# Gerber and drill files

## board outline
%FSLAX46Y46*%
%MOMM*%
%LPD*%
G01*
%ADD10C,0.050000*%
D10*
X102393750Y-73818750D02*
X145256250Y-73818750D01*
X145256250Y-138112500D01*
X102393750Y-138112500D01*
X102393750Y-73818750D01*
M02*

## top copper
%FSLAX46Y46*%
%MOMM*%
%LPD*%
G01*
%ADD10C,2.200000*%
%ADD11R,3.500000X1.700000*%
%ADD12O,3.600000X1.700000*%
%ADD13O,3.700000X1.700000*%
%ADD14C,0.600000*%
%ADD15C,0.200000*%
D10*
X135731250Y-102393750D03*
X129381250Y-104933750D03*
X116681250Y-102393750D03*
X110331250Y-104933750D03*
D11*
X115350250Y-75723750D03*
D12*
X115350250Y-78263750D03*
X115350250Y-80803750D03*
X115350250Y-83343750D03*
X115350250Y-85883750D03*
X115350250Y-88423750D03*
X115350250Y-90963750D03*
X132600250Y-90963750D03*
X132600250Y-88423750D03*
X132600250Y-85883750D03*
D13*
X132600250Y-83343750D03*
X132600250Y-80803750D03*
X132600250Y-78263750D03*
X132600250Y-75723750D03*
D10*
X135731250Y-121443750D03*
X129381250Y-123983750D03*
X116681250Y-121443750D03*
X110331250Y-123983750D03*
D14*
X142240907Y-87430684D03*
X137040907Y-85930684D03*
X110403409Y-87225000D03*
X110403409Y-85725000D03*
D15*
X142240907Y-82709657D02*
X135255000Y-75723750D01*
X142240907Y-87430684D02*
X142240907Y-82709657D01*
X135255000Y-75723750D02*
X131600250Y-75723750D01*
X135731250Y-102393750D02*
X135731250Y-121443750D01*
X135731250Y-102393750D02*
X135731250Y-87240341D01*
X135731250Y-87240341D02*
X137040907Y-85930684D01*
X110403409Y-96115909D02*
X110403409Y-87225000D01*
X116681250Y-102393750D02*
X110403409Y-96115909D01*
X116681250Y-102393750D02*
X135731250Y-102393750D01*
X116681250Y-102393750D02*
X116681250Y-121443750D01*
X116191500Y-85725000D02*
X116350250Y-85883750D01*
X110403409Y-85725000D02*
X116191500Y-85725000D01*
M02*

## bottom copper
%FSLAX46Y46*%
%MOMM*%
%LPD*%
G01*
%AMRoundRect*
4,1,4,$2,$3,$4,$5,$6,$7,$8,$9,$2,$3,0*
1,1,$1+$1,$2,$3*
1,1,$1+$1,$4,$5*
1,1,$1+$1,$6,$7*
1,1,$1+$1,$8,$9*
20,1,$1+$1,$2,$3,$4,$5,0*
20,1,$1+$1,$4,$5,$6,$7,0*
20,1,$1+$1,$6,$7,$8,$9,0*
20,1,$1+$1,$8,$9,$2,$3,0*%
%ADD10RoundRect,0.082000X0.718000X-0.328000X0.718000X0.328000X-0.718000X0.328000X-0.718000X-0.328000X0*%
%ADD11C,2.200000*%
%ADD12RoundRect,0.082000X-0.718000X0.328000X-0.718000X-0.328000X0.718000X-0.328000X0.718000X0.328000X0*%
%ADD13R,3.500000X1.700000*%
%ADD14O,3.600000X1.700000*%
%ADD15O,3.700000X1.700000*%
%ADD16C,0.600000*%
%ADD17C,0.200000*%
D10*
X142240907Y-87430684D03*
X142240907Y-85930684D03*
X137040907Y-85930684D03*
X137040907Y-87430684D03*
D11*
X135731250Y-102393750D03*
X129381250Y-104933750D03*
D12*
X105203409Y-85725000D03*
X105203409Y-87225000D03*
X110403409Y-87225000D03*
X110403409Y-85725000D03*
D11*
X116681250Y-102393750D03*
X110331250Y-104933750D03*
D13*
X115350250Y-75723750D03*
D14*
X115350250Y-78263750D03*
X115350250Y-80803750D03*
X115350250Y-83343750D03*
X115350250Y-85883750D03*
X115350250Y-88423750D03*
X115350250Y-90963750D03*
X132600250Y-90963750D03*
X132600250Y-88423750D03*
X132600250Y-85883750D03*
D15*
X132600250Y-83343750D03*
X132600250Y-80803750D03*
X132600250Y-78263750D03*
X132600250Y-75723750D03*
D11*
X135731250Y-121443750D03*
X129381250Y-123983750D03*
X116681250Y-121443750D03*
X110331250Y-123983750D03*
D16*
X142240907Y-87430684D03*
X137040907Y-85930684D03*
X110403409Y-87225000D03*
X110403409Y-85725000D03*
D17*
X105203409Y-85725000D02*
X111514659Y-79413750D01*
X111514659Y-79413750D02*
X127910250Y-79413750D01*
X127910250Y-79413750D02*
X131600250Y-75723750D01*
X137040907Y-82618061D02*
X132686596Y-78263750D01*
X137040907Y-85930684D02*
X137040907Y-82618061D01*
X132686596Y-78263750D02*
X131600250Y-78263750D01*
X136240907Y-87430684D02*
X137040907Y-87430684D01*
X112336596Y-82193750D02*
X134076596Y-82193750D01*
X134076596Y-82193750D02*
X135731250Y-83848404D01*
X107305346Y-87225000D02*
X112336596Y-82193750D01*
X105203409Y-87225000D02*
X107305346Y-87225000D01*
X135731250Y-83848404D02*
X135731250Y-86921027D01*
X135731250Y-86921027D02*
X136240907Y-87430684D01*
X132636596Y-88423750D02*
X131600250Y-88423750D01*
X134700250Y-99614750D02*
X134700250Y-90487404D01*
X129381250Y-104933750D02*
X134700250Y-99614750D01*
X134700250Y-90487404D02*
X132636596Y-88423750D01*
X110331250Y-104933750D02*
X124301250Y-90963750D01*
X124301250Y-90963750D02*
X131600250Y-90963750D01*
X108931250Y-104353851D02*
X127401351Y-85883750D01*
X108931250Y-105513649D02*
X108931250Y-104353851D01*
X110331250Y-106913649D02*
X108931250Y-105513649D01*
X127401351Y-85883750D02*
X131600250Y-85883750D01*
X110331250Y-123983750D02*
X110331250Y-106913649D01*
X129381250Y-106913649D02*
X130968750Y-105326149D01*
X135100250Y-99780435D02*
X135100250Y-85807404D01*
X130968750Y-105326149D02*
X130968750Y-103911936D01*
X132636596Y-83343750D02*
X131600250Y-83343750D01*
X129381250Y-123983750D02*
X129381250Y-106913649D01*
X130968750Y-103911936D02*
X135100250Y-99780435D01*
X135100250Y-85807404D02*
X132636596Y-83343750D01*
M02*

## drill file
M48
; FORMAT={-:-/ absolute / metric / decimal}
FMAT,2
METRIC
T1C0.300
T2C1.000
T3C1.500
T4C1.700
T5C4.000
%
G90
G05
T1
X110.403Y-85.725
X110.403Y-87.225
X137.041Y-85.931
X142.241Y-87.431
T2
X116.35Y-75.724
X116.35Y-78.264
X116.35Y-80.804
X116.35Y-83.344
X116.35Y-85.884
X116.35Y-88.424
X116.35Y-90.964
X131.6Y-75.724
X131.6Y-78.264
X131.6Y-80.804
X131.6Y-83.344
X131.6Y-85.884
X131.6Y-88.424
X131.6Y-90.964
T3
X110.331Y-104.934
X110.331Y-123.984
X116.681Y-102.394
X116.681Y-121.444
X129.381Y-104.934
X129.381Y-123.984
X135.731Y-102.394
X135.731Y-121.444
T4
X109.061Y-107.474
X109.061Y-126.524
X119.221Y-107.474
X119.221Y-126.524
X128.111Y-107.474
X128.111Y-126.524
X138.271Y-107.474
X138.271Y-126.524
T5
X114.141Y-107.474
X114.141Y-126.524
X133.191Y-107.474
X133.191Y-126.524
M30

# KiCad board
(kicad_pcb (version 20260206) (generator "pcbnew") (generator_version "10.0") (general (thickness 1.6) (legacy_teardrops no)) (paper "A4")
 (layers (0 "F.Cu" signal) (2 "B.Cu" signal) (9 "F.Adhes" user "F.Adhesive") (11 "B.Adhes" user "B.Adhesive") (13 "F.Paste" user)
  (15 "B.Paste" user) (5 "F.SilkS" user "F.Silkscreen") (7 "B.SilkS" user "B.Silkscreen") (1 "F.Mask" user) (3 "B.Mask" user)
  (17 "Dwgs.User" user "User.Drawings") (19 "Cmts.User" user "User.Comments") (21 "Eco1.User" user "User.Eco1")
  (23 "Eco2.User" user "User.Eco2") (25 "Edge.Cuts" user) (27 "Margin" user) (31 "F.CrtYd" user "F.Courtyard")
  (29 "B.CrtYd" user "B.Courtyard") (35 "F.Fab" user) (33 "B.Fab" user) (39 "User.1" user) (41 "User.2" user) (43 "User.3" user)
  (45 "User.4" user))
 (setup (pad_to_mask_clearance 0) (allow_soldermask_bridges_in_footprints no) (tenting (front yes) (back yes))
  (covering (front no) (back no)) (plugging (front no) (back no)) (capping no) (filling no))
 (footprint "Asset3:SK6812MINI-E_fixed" (layer "F.Cu") (at 139.640908 86.577842 180)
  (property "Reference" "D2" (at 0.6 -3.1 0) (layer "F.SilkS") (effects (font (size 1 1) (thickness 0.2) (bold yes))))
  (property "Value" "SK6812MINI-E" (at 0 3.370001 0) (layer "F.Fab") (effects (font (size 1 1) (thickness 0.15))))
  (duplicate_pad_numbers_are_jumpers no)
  (pad "1" smd roundrect (at -2.599999 -0.852842 90) (size 0.82 1.6) (layers "B.Cu" "B.Mask" "B.Paste") (roundrect_rratio 0.1) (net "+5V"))
  (pad "2" smd roundrect (at -2.599999 0.647158 90) (size 0.82 1.6) (layers "B.Cu" "B.Mask" "B.Paste") (roundrect_rratio 0.1)
   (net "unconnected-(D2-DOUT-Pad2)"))
  (pad "3" smd roundrect (at 2.600001 0.647158 90) (size 0.82 1.6) (layers "B.Cu" "B.Mask" "B.Paste") (roundrect_rratio 0.1) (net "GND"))
  (pad "4" smd roundrect (at 2.600001 -0.852842 90) (size 0.82 1.6) (layers "B.Cu" "B.Mask" "B.Paste") (roundrect_rratio 0.1)
   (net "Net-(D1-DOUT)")))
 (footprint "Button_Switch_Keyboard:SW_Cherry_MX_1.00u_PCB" (layer "F.Cu") (at 135.73125 102.39375)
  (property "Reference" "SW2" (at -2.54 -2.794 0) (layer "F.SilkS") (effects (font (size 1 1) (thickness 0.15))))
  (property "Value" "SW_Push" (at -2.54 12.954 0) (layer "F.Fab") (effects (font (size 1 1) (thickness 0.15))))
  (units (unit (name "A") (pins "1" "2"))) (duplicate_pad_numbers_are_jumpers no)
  (pad "" np_thru_hole circle (at -7.62 5.08) (size 1.7 1.7) (drill 1.7) (layers "*.Cu" "*.Mask"))
  (pad "" np_thru_hole circle (at -2.54 5.08) (size 4 4) (drill 4) (layers "*.Cu" "*.Mask"))
  (pad "" np_thru_hole circle (at 2.54 5.08) (size 1.7 1.7) (drill 1.7) (layers "*.Cu" "*.Mask"))
  (pad "1" thru_hole circle (at 0 0) (size 2.2 2.2) (drill 1.5) (layers "*.Cu" "*.Mask") (remove_unused_layers no) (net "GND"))
  (pad "2" thru_hole circle (at -6.35 2.54) (size 2.2 2.2) (drill 1.5) (layers "*.Cu" "*.Mask") (remove_unused_layers no)
   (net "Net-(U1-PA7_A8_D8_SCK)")))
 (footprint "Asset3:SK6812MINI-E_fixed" (layer "F.Cu") (at 107.803408 86.577842)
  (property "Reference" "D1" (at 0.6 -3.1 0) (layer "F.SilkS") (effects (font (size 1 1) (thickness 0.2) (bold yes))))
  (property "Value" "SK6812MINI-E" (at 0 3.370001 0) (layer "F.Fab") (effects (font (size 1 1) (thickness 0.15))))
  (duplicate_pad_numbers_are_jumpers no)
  (pad "1" smd roundrect (at -2.599999 -0.852842 270) (size 0.82 1.6) (layers "B.Cu" "B.Mask" "B.Paste") (roundrect_rratio 0.1) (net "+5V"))
  (pad "2" smd roundrect (at -2.599999 0.647158 270) (size 0.82 1.6) (layers "B.Cu" "B.Mask" "B.Paste") (roundrect_rratio 0.1)
   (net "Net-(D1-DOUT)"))
  (pad "3" smd roundrect (at 2.600001 0.647158 270) (size 0.82 1.6) (layers "B.Cu" "B.Mask" "B.Paste") (roundrect_rratio 0.1) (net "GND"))
  (pad "4" smd roundrect (at 2.600001 -0.852842 270) (size 0.82 1.6) (layers "B.Cu" "B.Mask" "B.Paste") (roundrect_rratio 0.1)
   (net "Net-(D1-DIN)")))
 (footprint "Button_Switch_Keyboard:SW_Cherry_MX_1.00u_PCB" (layer "F.Cu") (at 116.68125 102.39375)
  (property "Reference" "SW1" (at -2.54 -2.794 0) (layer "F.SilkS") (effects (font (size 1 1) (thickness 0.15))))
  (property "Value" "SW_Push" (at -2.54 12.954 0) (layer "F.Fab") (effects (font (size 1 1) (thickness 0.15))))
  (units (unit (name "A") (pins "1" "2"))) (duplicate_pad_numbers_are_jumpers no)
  (pad "" np_thru_hole circle (at -7.62 5.08) (size 1.7 1.7) (drill 1.7) (layers "*.Cu" "*.Mask"))
  (pad "" np_thru_hole circle (at -2.54 5.08) (size 4 4) (drill 4) (layers "*.Cu" "*.Mask"))
  (pad "" np_thru_hole circle (at 2.54 5.08) (size 1.7 1.7) (drill 1.7) (layers "*.Cu" "*.Mask"))
  (pad "1" thru_hole circle (at 0 0) (size 2.2 2.2) (drill 1.5) (layers "*.Cu" "*.Mask") (remove_unused_layers no) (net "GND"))
  (pad "2" thru_hole circle (at -6.35 2.54) (size 2.2 2.2) (drill 1.5) (layers "*.Cu" "*.Mask") (remove_unused_layers no)
   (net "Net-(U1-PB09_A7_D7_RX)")))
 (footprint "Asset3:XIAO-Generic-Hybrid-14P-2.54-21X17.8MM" (layer "F.Cu") (at 123.97525 83.34375)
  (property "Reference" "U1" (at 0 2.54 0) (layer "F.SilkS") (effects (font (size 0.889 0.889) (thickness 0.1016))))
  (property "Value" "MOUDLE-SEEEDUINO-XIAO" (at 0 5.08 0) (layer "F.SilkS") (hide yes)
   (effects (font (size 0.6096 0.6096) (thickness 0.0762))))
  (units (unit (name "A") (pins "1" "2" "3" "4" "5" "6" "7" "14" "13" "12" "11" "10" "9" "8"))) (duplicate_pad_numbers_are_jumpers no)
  (pad "1" thru_hole rect (at -7.625 -7.62) (size 3.5 1.7) (drill 1 (offset -1 0)) (layers "*.Cu" "*.Mask") (remove_unused_layers no)
   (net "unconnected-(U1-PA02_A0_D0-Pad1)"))
  (pad "2" thru_hole oval (at -7.625 -5.08) (size 3.6 1.7) (drill 1 (offset -1 0)) (layers "*.Cu" "*.Mask") (remove_unused_layers no)
   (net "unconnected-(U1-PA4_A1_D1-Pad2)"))
  (pad "3" thru_hole oval (at -7.625 -2.54) (size 3.6 1.7) (drill 1 (offset -1 0)) (layers "*.Cu" "*.Mask") (remove_unused_layers no)
   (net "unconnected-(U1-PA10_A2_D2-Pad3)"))
  (pad "4" thru_hole oval (at -7.625 0) (size 3.6 1.7) (drill 1 (offset -1 0)) (layers "*.Cu" "*.Mask") (remove_unused_layers no)
   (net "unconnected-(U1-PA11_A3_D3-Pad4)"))
  (pad "5" thru_hole oval (at -7.625 2.54) (size 3.6 1.7) (drill 1 (offset -1 0)) (layers "*.Cu" "*.Mask") (remove_unused_layers no)
   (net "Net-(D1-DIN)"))
  (pad "6" thru_hole oval (at -7.625 5.08 180) (size 3.6 1.7) (drill 1 (offset 1 0)) (layers "*.Cu" "*.Mask") (remove_unused_layers no)
   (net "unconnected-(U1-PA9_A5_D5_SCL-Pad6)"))
  (pad "7" thru_hole oval (at -7.625 7.62) (size 3.6 1.7) (drill 1 (offset -1 0)) (layers "*.Cu" "*.Mask") (remove_unused_layers no)
   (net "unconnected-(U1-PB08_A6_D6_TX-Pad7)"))
  (pad "8" thru_hole oval (at 7.625 7.62) (size 3.6 1.7) (drill 1 (offset 1 0)) (layers "*.Cu" "*.Mask") (remove_unused_layers no)
   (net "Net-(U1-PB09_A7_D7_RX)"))
  (pad "9" thru_hole oval (at 7.625 5.08) (size 3.6 1.7) (drill 1 (offset 1 0)) (layers "*.Cu" "*.Mask") (remove_unused_layers no)
   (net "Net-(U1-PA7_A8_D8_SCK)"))
  (pad "10" thru_hole oval (at 7.625 2.54) (size 3.6 1.7) (drill 1 (offset 1 0)) (layers "*.Cu" "*.Mask") (remove_unused_layers no)
   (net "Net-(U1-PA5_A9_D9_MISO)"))
  (pad "11" thru_hole oval (at 7.625 0) (size 3.7 1.7) (drill 1 (offset 1 0)) (layers "*.Cu" "*.Mask") (remove_unused_layers no)
   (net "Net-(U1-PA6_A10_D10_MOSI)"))
  (pad "12" thru_hole oval (at 7.625 -2.54) (size 3.7 1.7) (drill 1 (offset 1 0)) (layers "*.Cu" "*.Mask") (remove_unused_layers no)
   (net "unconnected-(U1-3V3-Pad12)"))
  (pad "13" thru_hole oval (at 7.625 -5.08) (size 3.7 1.7) (drill 1 (offset 1 0)) (layers "*.Cu" "*.Mask") (remove_unused_layers no)
   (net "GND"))
  (pad "14" thru_hole oval (at 7.625 -7.62) (size 3.7 1.7) (drill 1 (offset 1 0)) (layers "*.Cu" "*.Mask") (remove_unused_layers no)
   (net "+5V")))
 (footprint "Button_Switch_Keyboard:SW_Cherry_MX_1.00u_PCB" (layer "F.Cu") (at 135.73125 121.44375)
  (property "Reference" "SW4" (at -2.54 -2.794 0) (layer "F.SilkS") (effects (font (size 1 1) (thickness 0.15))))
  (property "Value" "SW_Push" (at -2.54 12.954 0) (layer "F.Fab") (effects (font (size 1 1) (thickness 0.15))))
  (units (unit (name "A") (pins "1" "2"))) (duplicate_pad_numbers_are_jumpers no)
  (pad "" np_thru_hole circle (at -7.62 5.08) (size 1.7 1.7) (drill 1.7) (layers "*.Cu" "*.Mask"))
  (pad "" np_thru_hole circle (at -2.54 5.08) (size 4 4) (drill 4) (layers "*.Cu" "*.Mask"))
  (pad "" np_thru_hole circle (at 2.54 5.08) (size 1.7 1.7) (drill 1.7) (layers "*.Cu" "*.Mask"))
  (pad "1" thru_hole circle (at 0 0) (size 2.2 2.2) (drill 1.5) (layers "*.Cu" "*.Mask") (remove_unused_layers no) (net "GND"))
  (pad "2" thru_hole circle (at -6.35 2.54) (size 2.2 2.2) (drill 1.5) (layers "*.Cu" "*.Mask") (remove_unused_layers no)
   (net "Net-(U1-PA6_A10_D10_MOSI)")))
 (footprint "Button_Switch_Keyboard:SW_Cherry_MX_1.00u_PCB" (layer "F.Cu") (at 116.68125 121.44375)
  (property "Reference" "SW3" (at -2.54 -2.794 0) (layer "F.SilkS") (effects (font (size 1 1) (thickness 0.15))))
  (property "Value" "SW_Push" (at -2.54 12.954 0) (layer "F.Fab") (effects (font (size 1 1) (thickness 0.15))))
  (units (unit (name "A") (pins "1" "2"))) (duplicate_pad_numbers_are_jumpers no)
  (pad "" np_thru_hole circle (at -7.62 5.08) (size 1.7 1.7) (drill 1.7) (layers "*.Cu" "*.Mask"))
  (pad "" np_thru_hole circle (at -2.54 5.08) (size 4 4) (drill 4) (layers "*.Cu" "*.Mask"))
  (pad "" np_thru_hole circle (at 2.54 5.08) (size 1.7 1.7) (drill 1.7) (layers "*.Cu" "*.Mask"))
  (pad "1" thru_hole circle (at 0 0) (size 2.2 2.2) (drill 1.5) (layers "*.Cu" "*.Mask") (remove_unused_layers no) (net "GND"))
  (pad "2" thru_hole circle (at -6.35 2.54) (size 2.2 2.2) (drill 1.5) (layers "*.Cu" "*.Mask") (remove_unused_layers no)
   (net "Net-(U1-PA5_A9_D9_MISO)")))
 (gr_rect (start 102.39375 73.81875) (end 145.25625 138.1125) (stroke (width 0.05) (type default)) (fill no) (layer "Edge.Cuts"))
 (segment (start 142.240907 82.709657) (end 135.255 75.72375) (width 0.2) (layer "F.Cu") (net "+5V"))
 (segment (start 142.240907 87.430684) (end 142.240907 82.709657) (width 0.2) (layer "F.Cu") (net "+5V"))
 (segment (start 135.255 75.72375) (end 131.60025 75.72375) (width 0.2) (layer "F.Cu") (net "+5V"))
 (via (at 142.240907 87.430684) (size 0.6) (drill 0.3) (layers "F.Cu" "B.Cu") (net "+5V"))
 (segment (start 105.203409 85.725) (end 111.514659 79.41375) (width 0.2) (layer "B.Cu") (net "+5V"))
 (segment (start 111.514659 79.41375) (end 127.91025 79.41375) (width 0.2) (layer "B.Cu") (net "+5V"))
 (segment (start 127.91025 79.41375) (end 131.60025 75.72375) (width 0.2) (layer "B.Cu") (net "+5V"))
 (segment (start 135.73125 102.39375) (end 135.73125 121.44375) (width 0.2) (layer "F.Cu") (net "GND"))
 (segment (start 135.73125 102.39375) (end 135.73125 87.240341) (width 0.2) (layer "F.Cu") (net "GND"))
 (segment (start 135.73125 87.240341) (end 137.040907 85.930684) (width 0.2) (layer "F.Cu") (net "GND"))
 (segment (start 110.403409 96.115909) (end 110.403409 87.225) (width 0.2) (layer "F.Cu") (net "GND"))
 (segment (start 116.68125 102.39375) (end 110.403409 96.115909) (width 0.2) (layer "F.Cu") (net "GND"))
 (segment (start 116.68125 102.39375) (end 135.73125 102.39375) (width 0.2) (layer "F.Cu") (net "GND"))
 (segment (start 116.68125 102.39375) (end 116.68125 121.44375) (width 0.2) (layer "F.Cu") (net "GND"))
 (via (at 137.040907 85.930684) (size 0.6) (drill 0.3) (layers "F.Cu" "B.Cu") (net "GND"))
 (via (at 110.403409 87.225) (size 0.6) (drill 0.3) (layers "F.Cu" "B.Cu") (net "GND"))
 (segment (start 137.040907 82.618061) (end 132.686596 78.26375) (width 0.2) (layer "B.Cu") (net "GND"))
 (segment (start 137.040907 85.930684) (end 137.040907 82.618061) (width 0.2) (layer "B.Cu") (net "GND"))
 (segment (start 132.686596 78.26375) (end 131.60025 78.26375) (width 0.2) (layer "B.Cu") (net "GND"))
 (segment (start 136.240907 87.430684) (end 137.040907 87.430684) (width 0.2) (layer "B.Cu") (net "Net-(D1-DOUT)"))
 (segment (start 112.336596 82.19375) (end 134.076596 82.19375) (width 0.2) (layer "B.Cu") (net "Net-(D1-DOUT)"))
 (segment (start 134.076596 82.19375) (end 135.73125 83.848404) (width 0.2) (layer "B.Cu") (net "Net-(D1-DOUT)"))
 (segment (start 107.305346 87.225) (end 112.336596 82.19375) (width 0.2) (layer "B.Cu") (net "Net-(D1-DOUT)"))
 (segment (start 105.203409 87.225) (end 107.305346 87.225) (width 0.2) (layer "B.Cu") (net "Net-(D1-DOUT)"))
 (segment (start 135.73125 83.848404) (end 135.73125 86.921027) (width 0.2) (layer "B.Cu") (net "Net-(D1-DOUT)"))
 (segment (start 135.73125 86.921027) (end 136.240907 87.430684) (width 0.2) (layer "B.Cu") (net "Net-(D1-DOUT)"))
 (segment (start 132.636596 88.42375) (end 131.60025 88.42375) (width 0.2) (layer "B.Cu") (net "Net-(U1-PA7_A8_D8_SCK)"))
 (segment (start 134.70025 99.61475) (end 134.70025 90.487404) (width 0.2) (layer "B.Cu") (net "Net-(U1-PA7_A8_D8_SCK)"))
 (segment (start 129.38125 104.93375) (end 134.70025 99.61475) (width 0.2) (layer "B.Cu") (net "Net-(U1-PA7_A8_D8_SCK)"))
 (segment (start 134.70025 90.487404) (end 132.636596 88.42375) (width 0.2) (layer "B.Cu") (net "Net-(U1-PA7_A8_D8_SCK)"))
 (segment (start 116.1915 85.725) (end 116.35025 85.88375) (width 0.2) (layer "F.Cu") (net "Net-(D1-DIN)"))
 (segment (start 110.403409 85.725) (end 116.1915 85.725) (width 0.2) (layer "F.Cu") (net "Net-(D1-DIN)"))
 (via (at 110.403409 85.725) (size 0.6) (drill 0.3) (layers "F.Cu" "B.Cu") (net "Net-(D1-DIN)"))
 (segment (start 110.33125 104.93375) (end 124.30125 90.96375) (width 0.2) (layer "B.Cu") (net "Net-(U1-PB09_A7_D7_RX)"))
 (segment (start 124.30125 90.96375) (end 131.60025 90.96375) (width 0.2) (layer "B.Cu") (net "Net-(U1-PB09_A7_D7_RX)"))
 (segment (start 108.93125 104.353851) (end 127.401351 85.88375) (width 0.2) (layer "B.Cu") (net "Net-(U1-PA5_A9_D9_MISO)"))
 (segment (start 108.93125 105.513649) (end 108.93125 104.353851) (width 0.2) (layer "B.Cu") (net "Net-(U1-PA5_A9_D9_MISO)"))
 (segment (start 110.33125 106.913649) (end 108.93125 105.513649) (width 0.2) (layer "B.Cu") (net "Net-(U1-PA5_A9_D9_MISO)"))
 (segment (start 127.401351 85.88375) (end 131.60025 85.88375) (width 0.2) (layer "B.Cu") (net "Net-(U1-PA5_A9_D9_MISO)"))
 (segment (start 110.33125 123.98375) (end 110.33125 106.913649) (width 0.2) (layer "B.Cu") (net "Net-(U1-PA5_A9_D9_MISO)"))
 (segment (start 129.38125 106.913649) (end 130.96875 105.326149) (width 0.2) (layer "B.Cu") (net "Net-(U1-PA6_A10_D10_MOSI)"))
 (segment (start 135.10025 99.780435) (end 135.10025 85.807404) (width 0.2) (layer "B.Cu") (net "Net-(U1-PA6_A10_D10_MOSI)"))
 (segment (start 130.96875 105.326149) (end 130.96875 103.911936) (width 0.2) (layer "B.Cu") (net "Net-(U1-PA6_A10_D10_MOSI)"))
 (segment (start 132.636596 83.34375) (end 131.60025 83.34375) (width 0.2) (layer "B.Cu") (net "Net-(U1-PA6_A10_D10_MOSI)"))
 (segment (start 129.38125 123.98375) (end 129.38125 106.913649) (width 0.2) (layer "B.Cu") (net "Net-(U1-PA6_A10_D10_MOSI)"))
 (segment (start 130.96875 103.911936) (end 135.10025 99.780435) (width 0.2) (layer "B.Cu") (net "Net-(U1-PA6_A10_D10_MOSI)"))
 (segment (start 135.10025 85.807404) (end 132.636596 83.34375) (width 0.2) (layer "B.Cu") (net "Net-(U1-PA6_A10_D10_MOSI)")))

